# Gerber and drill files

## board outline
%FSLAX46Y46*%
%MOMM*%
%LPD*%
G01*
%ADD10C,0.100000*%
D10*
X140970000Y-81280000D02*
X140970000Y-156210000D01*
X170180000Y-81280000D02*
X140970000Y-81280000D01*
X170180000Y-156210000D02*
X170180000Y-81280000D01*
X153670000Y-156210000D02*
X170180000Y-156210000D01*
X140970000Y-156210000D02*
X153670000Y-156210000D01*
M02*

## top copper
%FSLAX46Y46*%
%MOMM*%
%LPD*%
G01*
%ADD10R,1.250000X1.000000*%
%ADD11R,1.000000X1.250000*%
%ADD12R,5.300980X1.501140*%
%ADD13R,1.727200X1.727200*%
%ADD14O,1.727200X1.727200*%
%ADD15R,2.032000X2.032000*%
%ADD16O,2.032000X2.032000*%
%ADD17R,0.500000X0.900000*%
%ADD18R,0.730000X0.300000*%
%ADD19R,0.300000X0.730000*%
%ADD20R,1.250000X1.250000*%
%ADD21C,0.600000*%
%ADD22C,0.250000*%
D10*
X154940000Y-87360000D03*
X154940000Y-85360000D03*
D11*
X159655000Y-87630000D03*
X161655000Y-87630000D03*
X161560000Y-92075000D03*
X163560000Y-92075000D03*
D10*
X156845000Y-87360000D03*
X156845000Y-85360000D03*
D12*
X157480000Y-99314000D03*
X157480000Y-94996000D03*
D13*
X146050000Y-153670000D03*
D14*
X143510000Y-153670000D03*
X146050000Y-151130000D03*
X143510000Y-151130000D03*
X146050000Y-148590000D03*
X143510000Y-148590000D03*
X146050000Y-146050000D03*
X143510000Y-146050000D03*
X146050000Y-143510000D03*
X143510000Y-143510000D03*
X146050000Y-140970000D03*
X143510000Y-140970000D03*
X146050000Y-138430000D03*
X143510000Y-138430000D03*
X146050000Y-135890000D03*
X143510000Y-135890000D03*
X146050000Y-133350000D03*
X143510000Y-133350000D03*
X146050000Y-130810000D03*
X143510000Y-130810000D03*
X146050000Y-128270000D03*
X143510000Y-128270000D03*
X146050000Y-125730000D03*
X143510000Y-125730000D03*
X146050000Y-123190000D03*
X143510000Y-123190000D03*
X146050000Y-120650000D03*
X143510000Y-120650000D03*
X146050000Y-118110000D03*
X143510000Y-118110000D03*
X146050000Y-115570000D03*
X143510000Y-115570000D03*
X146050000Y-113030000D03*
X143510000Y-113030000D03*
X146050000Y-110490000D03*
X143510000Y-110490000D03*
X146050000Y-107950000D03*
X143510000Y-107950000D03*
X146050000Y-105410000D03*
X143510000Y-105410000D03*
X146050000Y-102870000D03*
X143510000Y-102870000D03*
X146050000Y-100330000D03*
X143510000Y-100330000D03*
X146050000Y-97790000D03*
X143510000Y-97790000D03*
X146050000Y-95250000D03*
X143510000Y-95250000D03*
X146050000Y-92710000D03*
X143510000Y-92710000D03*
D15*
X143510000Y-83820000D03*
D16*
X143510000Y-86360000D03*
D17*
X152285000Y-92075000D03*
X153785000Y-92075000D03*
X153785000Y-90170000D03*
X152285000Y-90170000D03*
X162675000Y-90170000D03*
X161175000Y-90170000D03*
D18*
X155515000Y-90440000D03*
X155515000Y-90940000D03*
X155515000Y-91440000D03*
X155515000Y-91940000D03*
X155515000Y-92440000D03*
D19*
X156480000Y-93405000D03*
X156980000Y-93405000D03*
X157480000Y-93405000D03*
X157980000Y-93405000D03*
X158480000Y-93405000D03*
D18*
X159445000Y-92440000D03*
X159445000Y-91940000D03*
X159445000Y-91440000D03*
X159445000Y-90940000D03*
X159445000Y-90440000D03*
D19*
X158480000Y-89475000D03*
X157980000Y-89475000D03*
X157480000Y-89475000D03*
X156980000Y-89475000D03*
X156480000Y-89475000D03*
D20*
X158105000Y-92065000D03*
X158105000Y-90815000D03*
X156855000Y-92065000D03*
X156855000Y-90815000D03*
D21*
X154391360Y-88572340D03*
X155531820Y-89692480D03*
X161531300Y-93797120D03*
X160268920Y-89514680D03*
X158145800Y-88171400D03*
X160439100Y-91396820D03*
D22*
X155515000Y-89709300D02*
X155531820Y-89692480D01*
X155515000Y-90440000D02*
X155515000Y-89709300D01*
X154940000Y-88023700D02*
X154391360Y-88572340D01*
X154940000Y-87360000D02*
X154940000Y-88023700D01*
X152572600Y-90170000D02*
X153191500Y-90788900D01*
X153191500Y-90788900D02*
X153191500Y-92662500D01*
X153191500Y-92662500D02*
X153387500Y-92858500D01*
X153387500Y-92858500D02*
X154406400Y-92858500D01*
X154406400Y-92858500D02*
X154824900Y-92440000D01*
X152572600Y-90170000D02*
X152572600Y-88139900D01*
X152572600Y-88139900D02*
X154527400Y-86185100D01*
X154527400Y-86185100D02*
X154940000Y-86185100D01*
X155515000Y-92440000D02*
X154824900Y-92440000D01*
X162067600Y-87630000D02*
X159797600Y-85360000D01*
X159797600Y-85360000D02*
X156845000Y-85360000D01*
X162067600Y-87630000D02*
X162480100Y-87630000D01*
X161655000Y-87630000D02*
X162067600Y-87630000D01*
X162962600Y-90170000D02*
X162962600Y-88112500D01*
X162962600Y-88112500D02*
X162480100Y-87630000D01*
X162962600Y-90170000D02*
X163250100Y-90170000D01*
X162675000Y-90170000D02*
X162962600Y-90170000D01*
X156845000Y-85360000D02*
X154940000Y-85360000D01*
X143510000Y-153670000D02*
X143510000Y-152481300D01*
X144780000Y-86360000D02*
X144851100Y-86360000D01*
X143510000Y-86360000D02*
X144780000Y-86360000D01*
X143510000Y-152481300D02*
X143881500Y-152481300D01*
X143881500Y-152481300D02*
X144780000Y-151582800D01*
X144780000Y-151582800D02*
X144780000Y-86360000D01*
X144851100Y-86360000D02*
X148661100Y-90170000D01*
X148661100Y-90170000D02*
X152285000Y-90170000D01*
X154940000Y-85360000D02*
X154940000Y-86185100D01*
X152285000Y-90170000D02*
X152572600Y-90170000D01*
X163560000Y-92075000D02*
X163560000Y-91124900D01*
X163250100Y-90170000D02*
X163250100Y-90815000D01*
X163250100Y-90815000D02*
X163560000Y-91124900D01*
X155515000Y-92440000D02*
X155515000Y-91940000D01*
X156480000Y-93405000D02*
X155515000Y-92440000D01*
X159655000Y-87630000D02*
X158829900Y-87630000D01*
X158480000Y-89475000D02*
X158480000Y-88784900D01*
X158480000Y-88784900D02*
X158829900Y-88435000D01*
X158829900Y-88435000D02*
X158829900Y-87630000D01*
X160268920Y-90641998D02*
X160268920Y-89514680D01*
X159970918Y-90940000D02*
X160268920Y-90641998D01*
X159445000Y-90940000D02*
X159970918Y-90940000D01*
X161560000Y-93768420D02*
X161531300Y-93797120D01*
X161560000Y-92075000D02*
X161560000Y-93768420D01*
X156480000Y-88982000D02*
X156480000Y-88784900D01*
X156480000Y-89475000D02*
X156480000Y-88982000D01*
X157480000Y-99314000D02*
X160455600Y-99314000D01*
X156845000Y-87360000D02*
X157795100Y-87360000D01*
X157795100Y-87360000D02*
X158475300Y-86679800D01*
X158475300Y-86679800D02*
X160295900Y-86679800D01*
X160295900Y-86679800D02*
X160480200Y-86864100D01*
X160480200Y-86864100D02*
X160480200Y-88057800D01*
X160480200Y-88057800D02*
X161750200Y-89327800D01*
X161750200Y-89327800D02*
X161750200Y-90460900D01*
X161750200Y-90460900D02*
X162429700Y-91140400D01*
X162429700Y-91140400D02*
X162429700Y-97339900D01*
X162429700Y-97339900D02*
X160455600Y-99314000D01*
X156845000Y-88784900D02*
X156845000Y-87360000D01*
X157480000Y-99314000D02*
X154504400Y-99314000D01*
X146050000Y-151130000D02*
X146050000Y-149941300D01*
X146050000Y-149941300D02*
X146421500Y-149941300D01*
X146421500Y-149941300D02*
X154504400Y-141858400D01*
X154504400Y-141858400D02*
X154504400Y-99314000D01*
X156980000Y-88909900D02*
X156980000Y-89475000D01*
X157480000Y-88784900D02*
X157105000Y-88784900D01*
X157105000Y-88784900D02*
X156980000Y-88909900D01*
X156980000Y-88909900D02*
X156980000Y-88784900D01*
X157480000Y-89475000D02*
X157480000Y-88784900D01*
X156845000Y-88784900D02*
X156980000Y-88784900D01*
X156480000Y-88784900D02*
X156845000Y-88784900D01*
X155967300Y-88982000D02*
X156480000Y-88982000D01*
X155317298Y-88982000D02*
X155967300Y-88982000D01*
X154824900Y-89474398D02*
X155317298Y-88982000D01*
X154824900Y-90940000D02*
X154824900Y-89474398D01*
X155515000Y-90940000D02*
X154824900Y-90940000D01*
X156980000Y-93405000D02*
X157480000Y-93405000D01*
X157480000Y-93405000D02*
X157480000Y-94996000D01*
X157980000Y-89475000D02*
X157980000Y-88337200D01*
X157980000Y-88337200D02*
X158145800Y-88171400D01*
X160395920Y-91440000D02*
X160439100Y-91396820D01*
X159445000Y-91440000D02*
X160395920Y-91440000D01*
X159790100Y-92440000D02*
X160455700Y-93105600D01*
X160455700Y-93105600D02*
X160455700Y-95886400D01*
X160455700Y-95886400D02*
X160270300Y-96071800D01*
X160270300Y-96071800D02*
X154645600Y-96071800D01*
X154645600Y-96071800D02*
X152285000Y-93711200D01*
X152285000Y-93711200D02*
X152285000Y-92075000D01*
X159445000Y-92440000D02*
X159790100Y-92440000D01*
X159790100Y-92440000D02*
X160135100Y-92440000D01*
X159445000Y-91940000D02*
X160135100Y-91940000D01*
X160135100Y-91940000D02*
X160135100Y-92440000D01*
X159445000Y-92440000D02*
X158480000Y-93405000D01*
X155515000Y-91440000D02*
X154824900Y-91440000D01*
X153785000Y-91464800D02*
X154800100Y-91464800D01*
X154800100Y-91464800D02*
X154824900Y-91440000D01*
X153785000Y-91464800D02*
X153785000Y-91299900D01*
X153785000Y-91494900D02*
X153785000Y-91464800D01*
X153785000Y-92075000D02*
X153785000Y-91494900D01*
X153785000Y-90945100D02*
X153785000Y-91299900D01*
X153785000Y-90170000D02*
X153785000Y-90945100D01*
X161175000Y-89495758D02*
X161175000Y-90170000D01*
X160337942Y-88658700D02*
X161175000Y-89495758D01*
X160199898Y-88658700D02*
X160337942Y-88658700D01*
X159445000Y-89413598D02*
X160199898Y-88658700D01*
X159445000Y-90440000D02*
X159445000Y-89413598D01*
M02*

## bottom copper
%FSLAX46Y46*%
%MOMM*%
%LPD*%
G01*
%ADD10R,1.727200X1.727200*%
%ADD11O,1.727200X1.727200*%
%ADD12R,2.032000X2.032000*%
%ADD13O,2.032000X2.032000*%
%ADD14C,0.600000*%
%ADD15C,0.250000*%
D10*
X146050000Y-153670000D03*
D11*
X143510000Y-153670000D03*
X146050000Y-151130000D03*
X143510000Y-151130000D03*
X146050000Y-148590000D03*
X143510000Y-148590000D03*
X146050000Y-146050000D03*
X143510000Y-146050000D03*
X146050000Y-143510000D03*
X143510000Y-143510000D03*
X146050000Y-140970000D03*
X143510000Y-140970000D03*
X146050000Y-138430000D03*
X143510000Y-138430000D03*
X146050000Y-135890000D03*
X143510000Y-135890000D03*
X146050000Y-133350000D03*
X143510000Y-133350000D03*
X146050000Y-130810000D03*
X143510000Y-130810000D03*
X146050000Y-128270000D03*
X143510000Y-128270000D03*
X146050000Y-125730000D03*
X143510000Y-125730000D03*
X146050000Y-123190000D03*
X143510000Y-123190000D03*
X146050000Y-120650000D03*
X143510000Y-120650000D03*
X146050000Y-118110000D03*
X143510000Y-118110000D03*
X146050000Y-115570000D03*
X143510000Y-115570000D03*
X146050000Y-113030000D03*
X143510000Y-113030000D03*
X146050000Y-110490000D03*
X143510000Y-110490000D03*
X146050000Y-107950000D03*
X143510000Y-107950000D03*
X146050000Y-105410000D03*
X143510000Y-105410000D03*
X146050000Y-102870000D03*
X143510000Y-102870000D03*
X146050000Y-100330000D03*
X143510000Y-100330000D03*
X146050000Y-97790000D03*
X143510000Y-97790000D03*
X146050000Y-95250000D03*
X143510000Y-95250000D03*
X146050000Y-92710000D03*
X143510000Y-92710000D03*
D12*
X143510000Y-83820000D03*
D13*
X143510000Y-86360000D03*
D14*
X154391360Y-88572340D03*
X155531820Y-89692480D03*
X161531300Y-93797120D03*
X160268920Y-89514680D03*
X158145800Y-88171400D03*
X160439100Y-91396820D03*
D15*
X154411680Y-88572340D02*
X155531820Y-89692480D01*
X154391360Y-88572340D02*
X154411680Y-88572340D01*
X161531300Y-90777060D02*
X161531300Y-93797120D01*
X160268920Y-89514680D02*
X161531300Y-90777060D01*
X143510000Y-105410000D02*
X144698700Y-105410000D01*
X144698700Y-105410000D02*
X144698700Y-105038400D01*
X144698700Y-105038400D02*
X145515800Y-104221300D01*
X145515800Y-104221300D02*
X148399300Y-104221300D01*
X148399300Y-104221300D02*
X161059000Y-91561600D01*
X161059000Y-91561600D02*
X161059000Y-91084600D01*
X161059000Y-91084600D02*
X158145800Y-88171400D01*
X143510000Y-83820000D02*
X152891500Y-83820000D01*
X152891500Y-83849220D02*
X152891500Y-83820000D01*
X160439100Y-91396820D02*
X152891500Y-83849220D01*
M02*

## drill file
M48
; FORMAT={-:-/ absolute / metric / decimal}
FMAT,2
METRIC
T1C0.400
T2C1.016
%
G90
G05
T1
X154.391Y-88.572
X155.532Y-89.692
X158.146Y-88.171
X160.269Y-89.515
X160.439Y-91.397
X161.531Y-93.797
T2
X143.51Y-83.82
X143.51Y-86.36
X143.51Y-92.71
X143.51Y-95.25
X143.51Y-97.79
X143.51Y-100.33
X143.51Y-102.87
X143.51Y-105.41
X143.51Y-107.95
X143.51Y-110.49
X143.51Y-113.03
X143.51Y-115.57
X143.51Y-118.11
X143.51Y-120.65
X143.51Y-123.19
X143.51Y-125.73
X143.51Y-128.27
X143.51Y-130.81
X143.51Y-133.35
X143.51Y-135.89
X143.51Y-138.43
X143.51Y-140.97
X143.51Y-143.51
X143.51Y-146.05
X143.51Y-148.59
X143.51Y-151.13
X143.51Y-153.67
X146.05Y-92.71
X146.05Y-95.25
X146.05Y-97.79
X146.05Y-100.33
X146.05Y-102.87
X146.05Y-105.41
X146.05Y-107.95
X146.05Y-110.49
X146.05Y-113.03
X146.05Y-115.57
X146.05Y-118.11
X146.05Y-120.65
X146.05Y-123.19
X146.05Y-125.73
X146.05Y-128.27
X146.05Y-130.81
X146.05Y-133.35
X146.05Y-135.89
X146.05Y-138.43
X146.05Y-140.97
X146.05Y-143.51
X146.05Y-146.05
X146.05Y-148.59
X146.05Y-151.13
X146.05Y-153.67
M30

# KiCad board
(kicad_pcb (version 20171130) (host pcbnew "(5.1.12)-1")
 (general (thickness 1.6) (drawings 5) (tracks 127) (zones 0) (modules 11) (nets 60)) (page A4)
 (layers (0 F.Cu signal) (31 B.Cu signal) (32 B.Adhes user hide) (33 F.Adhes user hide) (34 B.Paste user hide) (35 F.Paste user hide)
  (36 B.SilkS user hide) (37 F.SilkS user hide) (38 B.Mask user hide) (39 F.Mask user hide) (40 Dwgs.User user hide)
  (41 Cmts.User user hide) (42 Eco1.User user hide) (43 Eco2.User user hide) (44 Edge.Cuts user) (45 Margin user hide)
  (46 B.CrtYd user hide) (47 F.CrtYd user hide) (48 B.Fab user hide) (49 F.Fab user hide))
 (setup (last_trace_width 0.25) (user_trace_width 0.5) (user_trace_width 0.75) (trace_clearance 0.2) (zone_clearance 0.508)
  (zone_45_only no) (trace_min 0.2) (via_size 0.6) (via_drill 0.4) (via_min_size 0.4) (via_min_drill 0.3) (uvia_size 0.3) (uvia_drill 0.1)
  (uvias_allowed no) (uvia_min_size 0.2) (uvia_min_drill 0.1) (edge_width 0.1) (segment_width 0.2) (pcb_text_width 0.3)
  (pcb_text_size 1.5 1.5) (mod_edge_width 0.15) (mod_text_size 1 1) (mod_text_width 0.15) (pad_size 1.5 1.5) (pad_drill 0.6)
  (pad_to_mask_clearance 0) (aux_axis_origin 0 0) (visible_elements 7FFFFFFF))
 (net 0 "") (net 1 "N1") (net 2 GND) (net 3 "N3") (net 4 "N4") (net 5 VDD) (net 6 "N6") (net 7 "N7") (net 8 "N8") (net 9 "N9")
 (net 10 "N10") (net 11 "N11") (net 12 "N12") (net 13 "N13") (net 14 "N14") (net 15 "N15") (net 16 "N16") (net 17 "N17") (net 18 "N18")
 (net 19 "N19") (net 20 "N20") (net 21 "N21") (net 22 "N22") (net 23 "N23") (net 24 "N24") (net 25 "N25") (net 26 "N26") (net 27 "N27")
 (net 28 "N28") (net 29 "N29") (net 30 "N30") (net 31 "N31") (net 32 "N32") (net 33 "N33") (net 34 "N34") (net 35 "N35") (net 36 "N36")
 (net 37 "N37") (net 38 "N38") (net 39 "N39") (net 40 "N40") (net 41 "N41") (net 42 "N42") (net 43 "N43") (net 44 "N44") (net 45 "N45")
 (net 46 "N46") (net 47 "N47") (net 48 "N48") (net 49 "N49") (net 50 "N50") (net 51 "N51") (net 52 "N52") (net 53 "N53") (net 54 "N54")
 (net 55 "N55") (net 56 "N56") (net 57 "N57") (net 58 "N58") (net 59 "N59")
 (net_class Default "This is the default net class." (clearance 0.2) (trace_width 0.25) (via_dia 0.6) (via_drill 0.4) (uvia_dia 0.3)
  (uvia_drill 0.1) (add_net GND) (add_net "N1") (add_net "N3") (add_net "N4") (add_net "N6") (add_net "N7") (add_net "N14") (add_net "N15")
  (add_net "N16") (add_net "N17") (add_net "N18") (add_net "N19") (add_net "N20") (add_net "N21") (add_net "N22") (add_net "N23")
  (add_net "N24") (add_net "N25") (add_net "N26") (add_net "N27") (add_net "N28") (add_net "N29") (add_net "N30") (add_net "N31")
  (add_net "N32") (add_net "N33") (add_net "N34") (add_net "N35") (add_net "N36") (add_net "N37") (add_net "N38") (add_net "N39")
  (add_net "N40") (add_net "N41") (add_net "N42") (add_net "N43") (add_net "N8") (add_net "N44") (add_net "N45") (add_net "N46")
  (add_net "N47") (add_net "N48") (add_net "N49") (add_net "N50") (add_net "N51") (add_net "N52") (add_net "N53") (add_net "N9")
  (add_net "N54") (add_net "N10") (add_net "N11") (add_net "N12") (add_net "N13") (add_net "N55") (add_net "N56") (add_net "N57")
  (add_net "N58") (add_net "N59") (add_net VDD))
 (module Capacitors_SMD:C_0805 (layer F.Cu) (at 154.94 86.36 90)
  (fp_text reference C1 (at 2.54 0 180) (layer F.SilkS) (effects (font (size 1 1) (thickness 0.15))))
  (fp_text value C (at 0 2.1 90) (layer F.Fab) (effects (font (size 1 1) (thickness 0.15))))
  (pad 1 smd rect (at -1 0 90) (size 1 1.25) (layers F.Cu F.Paste F.Mask) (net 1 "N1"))
  (pad 2 smd rect (at 1 0 90) (size 1 1.25) (layers F.Cu F.Paste F.Mask) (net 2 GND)))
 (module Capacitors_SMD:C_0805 (layer F.Cu) (at 160.655 87.63)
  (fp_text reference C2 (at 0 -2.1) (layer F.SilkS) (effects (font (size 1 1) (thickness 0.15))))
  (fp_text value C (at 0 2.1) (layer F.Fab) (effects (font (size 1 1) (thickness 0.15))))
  (pad 1 smd rect (at -1 0) (size 1 1.25) (layers F.Cu F.Paste F.Mask) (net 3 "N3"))
  (pad 2 smd rect (at 1 0) (size 1 1.25) (layers F.Cu F.Paste F.Mask) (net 2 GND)))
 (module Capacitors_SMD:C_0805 (layer F.Cu) (at 162.56 92.075)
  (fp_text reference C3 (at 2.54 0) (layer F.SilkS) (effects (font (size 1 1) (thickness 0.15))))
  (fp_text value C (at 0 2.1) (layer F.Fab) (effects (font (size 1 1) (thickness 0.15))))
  (pad 1 smd rect (at -1 0) (size 1 1.25) (layers F.Cu F.Paste F.Mask) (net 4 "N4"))
  (pad 2 smd rect (at 1 0) (size 1 1.25) (layers F.Cu F.Paste F.Mask) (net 2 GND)))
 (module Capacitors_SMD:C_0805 (layer F.Cu) (at 156.845 86.36 90)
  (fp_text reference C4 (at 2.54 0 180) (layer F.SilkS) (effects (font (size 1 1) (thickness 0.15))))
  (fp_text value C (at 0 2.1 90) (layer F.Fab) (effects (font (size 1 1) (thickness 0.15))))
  (pad 1 smd rect (at -1 0 90) (size 1 1.25) (layers F.Cu F.Paste F.Mask) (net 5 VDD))
  (pad 2 smd rect (at 1 0 90) (size 1 1.25) (layers F.Cu F.Paste F.Mask) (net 2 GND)))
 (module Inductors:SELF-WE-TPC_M (layer F.Cu) (at 157.48 97.155 90)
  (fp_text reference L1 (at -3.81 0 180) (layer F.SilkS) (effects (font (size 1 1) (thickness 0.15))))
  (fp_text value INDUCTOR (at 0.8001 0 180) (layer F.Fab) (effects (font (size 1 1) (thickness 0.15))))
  (pad 1 smd rect (at -2.159 0 90) (size 1.50114 5.30098) (layers F.Cu F.Paste F.Mask) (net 5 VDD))
  (pad 2 smd rect (at 2.159 0 90) (size 1.50114 5.30098) (layers F.Cu F.Paste F.Mask) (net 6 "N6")))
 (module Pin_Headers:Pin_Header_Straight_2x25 (layer F.Cu) (at 146.05 153.67 180)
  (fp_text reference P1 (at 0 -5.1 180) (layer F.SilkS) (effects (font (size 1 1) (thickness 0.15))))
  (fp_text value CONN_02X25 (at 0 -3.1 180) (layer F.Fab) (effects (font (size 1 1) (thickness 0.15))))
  (pad 1 thru_hole rect (at 0 0 180) (size 1.7272 1.7272) (drill 1.016) (layers *.Cu *.Mask F.SilkS) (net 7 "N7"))
  (pad 2 thru_hole oval (at 2.54 0 180) (size 1.7272 1.7272) (drill 1.016) (layers *.Cu *.Mask F.SilkS) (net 2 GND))
  (pad 3 thru_hole oval (at 0 2.54 180) (size 1.7272 1.7272) (drill 1.016) (layers *.Cu *.Mask F.SilkS) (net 5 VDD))
  (pad 4 thru_hole oval (at 2.54 2.54 180) (size 1.7272 1.7272) (drill 1.016) (layers *.Cu *.Mask F.SilkS) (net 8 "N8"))
  (pad 5 thru_hole oval (at 0 5.08 180) (size 1.7272 1.7272) (drill 1.016) (layers *.Cu *.Mask F.SilkS) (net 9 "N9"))
  (pad 6 thru_hole oval (at 2.54 5.08 180) (size 1.7272 1.7272) (drill 1.016) (layers *.Cu *.Mask F.SilkS) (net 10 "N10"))
  (pad 7 thru_hole oval (at 0 7.62 180) (size 1.7272 1.7272) (drill 1.016) (layers *.Cu *.Mask F.SilkS) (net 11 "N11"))
  (pad 8 thru_hole oval (at 2.54 7.62 180) (size 1.7272 1.7272) (drill 1.016) (layers *.Cu *.Mask F.SilkS) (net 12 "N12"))
  (pad 9 thru_hole oval (at 0 10.16 180) (size 1.7272 1.7272) (drill 1.016) (layers *.Cu *.Mask F.SilkS) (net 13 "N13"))
  (pad 10 thru_hole oval (at 2.54 10.16 180) (size 1.7272 1.7272) (drill 1.016) (layers *.Cu *.Mask F.SilkS) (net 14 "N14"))
  (pad 11 thru_hole oval (at 0 12.7 180) (size 1.7272 1.7272) (drill 1.016) (layers *.Cu *.Mask F.SilkS) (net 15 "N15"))
  (pad 12 thru_hole oval (at 2.54 12.7 180) (size 1.7272 1.7272) (drill 1.016) (layers *.Cu *.Mask F.SilkS) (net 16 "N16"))
  (pad 13 thru_hole oval (at 0 15.24 180) (size 1.7272 1.7272) (drill 1.016) (layers *.Cu *.Mask F.SilkS) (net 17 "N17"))
  (pad 14 thru_hole oval (at 2.54 15.24 180) (size 1.7272 1.7272) (drill 1.016) (layers *.Cu *.Mask F.SilkS) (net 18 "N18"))
  (pad 15 thru_hole oval (at 0 17.78 180) (size 1.7272 1.7272) (drill 1.016) (layers *.Cu *.Mask F.SilkS) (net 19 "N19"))
  (pad 16 thru_hole oval (at 2.54 17.78 180) (size 1.7272 1.7272) (drill 1.016) (layers *.Cu *.Mask F.SilkS) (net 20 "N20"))
  (pad 17 thru_hole oval (at 0 20.32 180) (size 1.7272 1.7272) (drill 1.016) (layers *.Cu *.Mask F.SilkS) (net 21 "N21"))
  (pad 18 thru_hole oval (at 2.54 20.32 180) (size 1.7272 1.7272) (drill 1.016) (layers *.Cu *.Mask F.SilkS) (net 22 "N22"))
  (pad 19 thru_hole oval (at 0 22.86 180) (size 1.7272 1.7272) (drill 1.016) (layers *.Cu *.Mask F.SilkS) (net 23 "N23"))
  (pad 20 thru_hole oval (at 2.54 22.86 180) (size 1.7272 1.7272) (drill 1.016) (layers *.Cu *.Mask F.SilkS) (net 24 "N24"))
  (pad 21 thru_hole oval (at 0 25.4 180) (size 1.7272 1.7272) (drill 1.016) (layers *.Cu *.Mask F.SilkS) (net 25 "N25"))
  (pad 22 thru_hole oval (at 2.54 25.4 180) (size 1.7272 1.7272) (drill 1.016) (layers *.Cu *.Mask F.SilkS) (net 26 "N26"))
  (pad 23 thru_hole oval (at 0 27.94 180) (size 1.7272 1.7272) (drill 1.016) (layers *.Cu *.Mask F.SilkS) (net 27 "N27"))
  (pad 24 thru_hole oval (at 2.54 27.94 180) (size 1.7272 1.7272) (drill 1.016) (layers *.Cu *.Mask F.SilkS) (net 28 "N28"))
  (pad 25 thru_hole oval (at 0 30.48 180) (size 1.7272 1.7272) (drill 1.016) (layers *.Cu *.Mask F.SilkS) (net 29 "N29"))
  (pad 26 thru_hole oval (at 2.54 30.48 180) (size 1.7272 1.7272) (drill 1.016) (layers *.Cu *.Mask F.SilkS) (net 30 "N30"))
  (pad 27 thru_hole oval (at 0 33.02 180) (size 1.7272 1.7272) (drill 1.016) (layers *.Cu *.Mask F.SilkS) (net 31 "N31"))
  (pad 28 thru_hole oval (at 2.54 33.02 180) (size 1.7272 1.7272) (drill 1.016) (layers *.Cu *.Mask F.SilkS) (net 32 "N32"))
  (pad 29 thru_hole oval (at 0 35.56 180) (size 1.7272 1.7272) (drill 1.016) (layers *.Cu *.Mask F.SilkS) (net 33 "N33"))
  (pad 30 thru_hole oval (at 2.54 35.56 180) (size 1.7272 1.7272) (drill 1.016) (layers *.Cu *.Mask F.SilkS) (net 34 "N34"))
  (pad 31 thru_hole oval (at 0 38.1 180) (size 1.7272 1.7272) (drill 1.016) (layers *.Cu *.Mask F.SilkS) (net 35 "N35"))
  (pad 32 thru_hole oval (at 2.54 38.1 180) (size 1.7272 1.7272) (drill 1.016) (layers *.Cu *.Mask F.SilkS) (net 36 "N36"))
  (pad 33 thru_hole oval (at 0 40.64 180) (size 1.7272 1.7272) (drill 1.016) (layers *.Cu *.Mask F.SilkS) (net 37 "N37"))
  (pad 34 thru_hole oval (at 2.54 40.64 180) (size 1.7272 1.7272) (drill 1.016) (layers *.Cu *.Mask F.SilkS) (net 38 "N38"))
  (pad 35 thru_hole oval (at 0 43.18 180) (size 1.7272 1.7272) (drill 1.016) (layers *.Cu *.Mask F.SilkS) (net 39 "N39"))
  (pad 36 thru_hole oval (at 2.54 43.18 180) (size 1.7272 1.7272) (drill 1.016) (layers *.Cu *.Mask F.SilkS) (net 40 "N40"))
  (pad 37 thru_hole oval (at 0 45.72 180) (size 1.7272 1.7272) (drill 1.016) (layers *.Cu *.Mask F.SilkS) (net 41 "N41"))
  (pad 38 thru_hole oval (at 2.54 45.72 180) (size 1.7272 1.7272) (drill 1.016) (layers *.Cu *.Mask F.SilkS) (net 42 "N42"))
  (pad 39 thru_hole oval (at 0 48.26 180) (size 1.7272 1.7272) (drill 1.016) (layers *.Cu *.Mask F.SilkS) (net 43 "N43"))
  (pad 40 thru_hole oval (at 2.54 48.26 180) (size 1.7272 1.7272) (drill 1.016) (layers *.Cu *.Mask F.SilkS) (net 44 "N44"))
  (pad 41 thru_hole oval (at 0 50.8 180) (size 1.7272 1.7272) (drill 1.016) (layers *.Cu *.Mask F.SilkS) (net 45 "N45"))
  (pad 42 thru_hole oval (at 2.54 50.8 180) (size 1.7272 1.7272) (drill 1.016) (layers *.Cu *.Mask F.SilkS) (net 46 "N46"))
  (pad 43 thru_hole oval (at 0 53.34 180) (size 1.7272 1.7272) (drill 1.016) (layers *.Cu *.Mask F.SilkS) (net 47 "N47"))
  (pad 44 thru_hole oval (at 2.54 53.34 180) (size 1.7272 1.7272) (drill 1.016) (layers *.Cu *.Mask F.SilkS) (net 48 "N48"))
  (pad 45 thru_hole oval (at 0 55.88 180) (size 1.7272 1.7272) (drill 1.016) (layers *.Cu *.Mask F.SilkS) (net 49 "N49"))
  (pad 46 thru_hole oval (at 2.54 55.88 180) (size 1.7272 1.7272) (drill 1.016) (layers *.Cu *.Mask F.SilkS) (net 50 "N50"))
  (pad 47 thru_hole oval (at 0 58.42 180) (size 1.7272 1.7272) (drill 1.016) (layers *.Cu *.Mask F.SilkS) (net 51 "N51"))
  (pad 48 thru_hole oval (at 2.54 58.42 180) (size 1.7272 1.7272) (drill 1.016) (layers *.Cu *.Mask F.SilkS) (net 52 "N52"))
  (pad 49 thru_hole oval (at 0 60.96 180) (size 1.7272 1.7272) (drill 1.016) (layers *.Cu *.Mask F.SilkS) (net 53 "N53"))
  (pad 50 thru_hole oval (at 2.54 60.96 180) (size 1.7272 1.7272) (drill 1.016) (layers *.Cu *.Mask F.SilkS) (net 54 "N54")))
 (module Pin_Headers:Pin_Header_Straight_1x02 (layer F.Cu) (at 143.51 83.82)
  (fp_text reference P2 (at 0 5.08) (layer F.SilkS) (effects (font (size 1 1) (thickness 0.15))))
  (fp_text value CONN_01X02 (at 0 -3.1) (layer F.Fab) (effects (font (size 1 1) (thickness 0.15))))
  (pad 1 thru_hole rect (at 0 0) (size 2.032 2.032) (drill 1.016) (layers *.Cu *.Mask F.SilkS) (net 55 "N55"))
  (pad 2 thru_hole oval (at 0 2.54) (size 2.032 2.032) (drill 1.016) (layers *.Cu *.Mask F.SilkS) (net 2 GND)))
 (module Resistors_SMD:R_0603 (layer F.Cu) (at 153.035 92.075)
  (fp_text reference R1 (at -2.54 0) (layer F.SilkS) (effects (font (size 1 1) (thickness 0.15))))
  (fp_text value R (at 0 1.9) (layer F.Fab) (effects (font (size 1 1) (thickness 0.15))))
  (pad 1 smd rect (at -0.75 0) (size 0.5 0.9) (layers F.Cu F.Paste F.Mask) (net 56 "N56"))
  (pad 2 smd rect (at 0.75 0) (size 0.5 0.9) (layers F.Cu F.Paste F.Mask) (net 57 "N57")))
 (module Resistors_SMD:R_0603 (layer F.Cu) (at 153.035 90.17 180)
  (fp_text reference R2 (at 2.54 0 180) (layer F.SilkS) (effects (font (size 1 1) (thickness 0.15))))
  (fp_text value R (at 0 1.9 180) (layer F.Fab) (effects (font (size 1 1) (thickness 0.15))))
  (pad 1 smd rect (at -0.75 0 180) (size 0.5 0.9) (layers F.Cu F.Paste F.Mask) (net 57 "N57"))
  (pad 2 smd rect (at 0.75 0 180) (size 0.5 0.9) (layers F.Cu F.Paste F.Mask) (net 2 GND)))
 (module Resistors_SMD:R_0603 (layer F.Cu) (at 161.925 90.17 180)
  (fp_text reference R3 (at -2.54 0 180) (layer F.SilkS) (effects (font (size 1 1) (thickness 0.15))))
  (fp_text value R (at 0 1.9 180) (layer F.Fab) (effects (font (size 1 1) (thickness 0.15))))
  (pad 1 smd rect (at -0.75 0 180) (size 0.5 0.9) (layers F.Cu F.Paste F.Mask) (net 2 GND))
  (pad 2 smd rect (at 0.75 0 180) (size 0.5 0.9) (layers F.Cu F.Paste F.Mask) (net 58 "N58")))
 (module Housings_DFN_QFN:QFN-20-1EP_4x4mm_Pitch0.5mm (layer F.Cu) (at 157.48 91.44)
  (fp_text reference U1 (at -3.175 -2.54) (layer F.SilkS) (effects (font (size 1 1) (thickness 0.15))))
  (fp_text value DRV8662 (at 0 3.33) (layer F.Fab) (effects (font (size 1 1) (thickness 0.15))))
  (pad 1 smd rect (at -1.965 -1) (size 0.73 0.3) (layers F.Cu F.Paste F.Mask) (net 1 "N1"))
  (pad 2 smd rect (at -1.965 -0.5) (size 0.73 0.3) (layers F.Cu F.Paste F.Mask) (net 5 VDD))
  (pad 3 smd rect (at -1.965 0) (size 0.73 0.3) (layers F.Cu F.Paste F.Mask) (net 57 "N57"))
  (pad 4 smd rect (at -1.965 0.5) (size 0.73 0.3) (layers F.Cu F.Paste F.Mask) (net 2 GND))
  (pad 5 smd rect (at -1.965 1) (size 0.73 0.3) (layers F.Cu F.Paste F.Mask) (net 2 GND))
  (pad 6 smd rect (at -1 1.965 90) (size 0.73 0.3) (layers F.Cu F.Paste F.Mask) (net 2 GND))
  (pad 7 smd rect (at -0.5 1.965 90) (size 0.73 0.3) (layers F.Cu F.Paste F.Mask) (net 6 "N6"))
  (pad 8 smd rect (at 0 1.965 90) (size 0.73 0.3) (layers F.Cu F.Paste F.Mask) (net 6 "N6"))
  (pad 9 smd rect (at 0.5 1.965 90) (size 0.73 0.3) (layers F.Cu F.Paste F.Mask) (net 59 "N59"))
  (pad 10 smd rect (at 1 1.965 90) (size 0.73 0.3) (layers F.Cu F.Paste F.Mask) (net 56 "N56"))
  (pad 11 smd rect (at 1.965 1) (size 0.73 0.3) (layers F.Cu F.Paste F.Mask) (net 56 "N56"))
  (pad 12 smd rect (at 1.965 0.5) (size 0.73 0.3) (layers F.Cu F.Paste F.Mask) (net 56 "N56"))
  (pad 13 smd rect (at 1.965 0) (size 0.73 0.3) (layers F.Cu F.Paste F.Mask) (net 55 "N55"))
  (pad 14 smd rect (at 1.965 -0.5) (size 0.73 0.3) (layers F.Cu F.Paste F.Mask) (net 4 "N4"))
  (pad 15 smd rect (at 1.965 -1) (size 0.73 0.3) (layers F.Cu F.Paste F.Mask) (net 58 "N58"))
  (pad 16 smd rect (at 1 -1.965 90) (size 0.73 0.3) (layers F.Cu F.Paste F.Mask) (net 3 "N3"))
  (pad 17 smd rect (at 0.5 -1.965 90) (size 0.73 0.3) (layers F.Cu F.Paste F.Mask) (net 44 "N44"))
  (pad 18 smd rect (at 0 -1.965 90) (size 0.73 0.3) (layers F.Cu F.Paste F.Mask) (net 5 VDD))
  (pad 19 smd rect (at -0.5 -1.965 90) (size 0.73 0.3) (layers F.Cu F.Paste F.Mask) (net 5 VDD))
  (pad 20 smd rect (at -1 -1.965 90) (size 0.73 0.3) (layers F.Cu F.Paste F.Mask) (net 5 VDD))
  (pad 21 smd rect (at 0.625 0.625) (size 1.25 1.25) (layers F.Cu F.Paste F.Mask) (solder_paste_margin_ratio -0.2))
  (pad 21 smd rect (at 0.625 -0.625) (size 1.25 1.25) (layers F.Cu F.Paste F.Mask) (solder_paste_margin_ratio -0.2))
  (pad 21 smd rect (at -0.625 0.625) (size 1.25 1.25) (layers F.Cu F.Paste F.Mask) (solder_paste_margin_ratio -0.2))
  (pad 21 smd rect (at -0.625 -0.625) (size 1.25 1.25) (layers F.Cu F.Paste F.Mask) (solder_paste_margin_ratio -0.2)))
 (gr_line (start 140.97 81.28) (end 140.97 156.21) (angle 90) (layer Edge.Cuts) (width 0.1))
 (gr_line (start 170.18 81.28) (end 140.97 81.28) (angle 90) (layer Edge.Cuts) (width 0.1))
 (gr_line (start 170.18 156.21) (end 170.18 81.28) (angle 90) (layer Edge.Cuts) (width 0.1))
 (gr_line (start 153.67 156.21) (end 170.18 156.21) (angle 90) (layer Edge.Cuts) (width 0.1))
 (gr_line (start 140.97 156.21) (end 153.67 156.21) (angle 90) (layer Edge.Cuts) (width 0.1))
 (via (at 154.39136 88.57234) (size 0.6) (drill 0.4) (layers F.Cu B.Cu) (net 1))
 (via (at 155.53182 89.69248) (size 0.6) (drill 0.4) (layers F.Cu B.Cu) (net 1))
 (segment (start 155.515 89.7093) (end 155.53182 89.69248) (width 0.25) (layer F.Cu) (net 1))
 (segment (start 155.515 90.44) (end 155.515 89.7093) (width 0.25) (layer F.Cu) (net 1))
 (segment (start 154.94 88.0237) (end 154.39136 88.57234) (width 0.25) (layer F.Cu) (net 1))
 (segment (start 154.94 87.36) (end 154.94 88.0237) (width 0.25) (layer F.Cu) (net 1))
 (segment (start 154.41168 88.57234) (end 155.53182 89.69248) (width 0.25) (layer B.Cu) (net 1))
 (segment (start 154.39136 88.57234) (end 154.41168 88.57234) (width 0.25) (layer B.Cu) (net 1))
 (via (at 161.5313 93.79712) (size 0.6) (drill 0.4) (layers F.Cu B.Cu) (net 4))
 (via (at 160.26892 89.51468) (size 0.6) (drill 0.4) (layers F.Cu B.Cu) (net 4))
 (segment (start 152.5726 90.17) (end 153.1915 90.7889) (width 0.25) (layer F.Cu) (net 2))
 (segment (start 153.1915 90.7889) (end 153.1915 92.6625) (width 0.25) (layer F.Cu) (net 2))
 (segment (start 153.1915 92.6625) (end 153.3875 92.8585) (width 0.25) (layer F.Cu) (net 2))
 (segment (start 153.3875 92.8585) (end 154.4064 92.8585) (width 0.25) (layer F.Cu) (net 2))
 (segment (start 154.4064 92.8585) (end 154.8249 92.44) (width 0.25) (layer F.Cu) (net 2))
 (segment (start 152.5726 90.17) (end 152.5726 88.1399) (width 0.25) (layer F.Cu) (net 2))
 (segment (start 152.5726 88.1399) (end 154.5274 86.1851) (width 0.25) (layer F.Cu) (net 2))
 (segment (start 154.5274 86.1851) (end 154.94 86.1851) (width 0.25) (layer F.Cu) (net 2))
 (segment (start 155.515 92.44) (end 154.8249 92.44) (width 0.25) (layer F.Cu) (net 2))
 (segment (start 162.0676 87.63) (end 159.7976 85.36) (width 0.25) (layer F.Cu) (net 2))
 (segment (start 159.7976 85.36) (end 156.845 85.36) (width 0.25) (layer F.Cu) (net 2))
 (segment (start 162.0676 87.63) (end 162.4801 87.63) (width 0.25) (layer F.Cu) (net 2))
 (segment (start 161.655 87.63) (end 162.0676 87.63) (width 0.25) (layer F.Cu) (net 2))
 (segment (start 162.9626 90.17) (end 162.9626 88.1125) (width 0.25) (layer F.Cu) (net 2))
 (segment (start 162.9626 88.1125) (end 162.4801 87.63) (width 0.25) (layer F.Cu) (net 2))
 (segment (start 162.9626 90.17) (end 163.2501 90.17) (width 0.25) (layer F.Cu) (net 2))
 (segment (start 162.675 90.17) (end 162.9626 90.17) (width 0.25) (layer F.Cu) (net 2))
 (segment (start 156.845 85.36) (end 154.94 85.36) (width 0.25) (layer F.Cu) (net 2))
 (segment (start 143.51 153.67) (end 143.51 152.4813) (width 0.25) (layer F.Cu) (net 2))
 (segment (start 144.78 86.36) (end 144.8511 86.36) (width 0.25) (layer F.Cu) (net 2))
 (segment (start 143.51 86.36) (end 144.78 86.36) (width 0.25) (layer F.Cu) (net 2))
 (segment (start 143.51 152.4813) (end 143.8815 152.4813) (width 0.25) (layer F.Cu) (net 2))
 (segment (start 143.8815 152.4813) (end 144.78 151.5828) (width 0.25) (layer F.Cu) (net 2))
 (segment (start 144.78 151.5828) (end 144.78 86.36) (width 0.25) (layer F.Cu) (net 2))
 (segment (start 144.8511 86.36) (end 148.6611 90.17) (width 0.25) (layer F.Cu) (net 2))
 (segment (start 148.6611 90.17) (end 152.285 90.17) (width 0.25) (layer F.Cu) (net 2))
 (segment (start 154.94 85.36) (end 154.94 86.1851) (width 0.25) (layer F.Cu) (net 2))
 (segment (start 152.285 90.17) (end 152.5726 90.17) (width 0.25) (layer F.Cu) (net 2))
 (segment (start 163.56 92.075) (end 163.56 91.1249) (width 0.25) (layer F.Cu) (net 2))
 (segment (start 163.2501 90.17) (end 163.2501 90.815) (width 0.25) (layer F.Cu) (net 2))
 (segment (start 163.2501 90.815) (end 163.56 91.1249) (width 0.25) (layer F.Cu) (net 2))
 (segment (start 155.515 92.44) (end 155.515 91.94) (width 0.25) (layer F.Cu) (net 2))
 (segment (start 156.48 93.405) (end 155.515 92.44) (width 0.25) (layer F.Cu) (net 2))
 (segment (start 159.655 87.63) (end 158.8299 87.63) (width 0.25) (layer F.Cu) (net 3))
 (segment (start 158.48 89.475) (end 158.48 88.7849) (width 0.25) (layer F.Cu) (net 3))
 (segment (start 158.48 88.7849) (end 158.8299 88.435) (width 0.25) (layer F.Cu) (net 3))
 (segment (start 158.8299 88.435) (end 158.8299 87.63) (width 0.25) (layer F.Cu) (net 3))
 (segment (start 160.26892 90.641998) (end 160.26892 89.51468) (width 0.25) (layer F.Cu) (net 4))
 (segment (start 159.970918 90.94) (end 160.26892 90.641998) (width 0.25) (layer F.Cu) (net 4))
 (segment (start 159.445 90.94) (end 159.970918 90.94) (width 0.25) (layer F.Cu) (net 4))
 (segment (start 161.56 93.76842) (end 161.5313 93.79712) (width 0.25) (layer F.Cu) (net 4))
 (segment (start 161.56 92.075) (end 161.56 93.76842) (width 0.25) (layer F.Cu) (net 4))
 (segment (start 161.5313 90.77706) (end 161.5313 93.79712) (width 0.25) (layer B.Cu) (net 4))
 (segment (start 160.26892 89.51468) (end 161.5313 90.77706) (width 0.25) (layer B.Cu) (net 4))
 (segment (start 156.48 88.982) (end 156.48 88.7849) (width 0.25) (layer F.Cu) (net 5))
 (segment (start 156.48 89.475) (end 156.48 88.982) (width 0.25) (layer F.Cu) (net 5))
 (segment (start 157.48 99.314) (end 160.4556 99.314) (width 0.25) (layer F.Cu) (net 5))
 (segment (start 156.845 87.36) (end 157.7951 87.36) (width 0.25) (layer F.Cu) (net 5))
 (segment (start 157.7951 87.36) (end 158.4753 86.6798) (width 0.25) (layer F.Cu) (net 5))
 (segment (start 158.4753 86.6798) (end 160.2959 86.6798) (width 0.25) (layer F.Cu) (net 5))
 (segment (start 160.2959 86.6798) (end 160.4802 86.8641) (width 0.25) (layer F.Cu) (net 5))
 (segment (start 160.4802 86.8641) (end 160.4802 88.0578) (width 0.25) (layer F.Cu) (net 5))
 (segment (start 160.4802 88.0578) (end 161.7502 89.3278) (width 0.25) (layer F.Cu) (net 5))
 (segment (start 161.7502 89.3278) (end 161.7502 90.4609) (width 0.25) (layer F.Cu) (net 5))
 (segment (start 161.7502 90.4609) (end 162.4297 91.1404) (width 0.25) (layer F.Cu) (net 5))
 (segment (start 162.4297 91.1404) (end 162.4297 97.3399) (width 0.25) (layer F.Cu) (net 5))
 (segment (start 162.4297 97.3399) (end 160.4556 99.314) (width 0.25) (layer F.Cu) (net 5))
 (segment (start 156.845 88.7849) (end 156.845 87.36) (width 0.25) (layer F.Cu) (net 5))
 (segment (start 157.48 99.314) (end 154.5044 99.314) (width 0.25) (layer F.Cu) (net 5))
 (segment (start 146.05 151.13) (end 146.05 149.9413) (width 0.25) (layer F.Cu) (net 5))
 (segment (start 146.05 149.9413) (end 146.4215 149.9413) (width 0.25) (layer F.Cu) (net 5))
 (segment (start 146.4215 149.9413) (end 154.5044 141.8584) (width 0.25) (layer F.Cu) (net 5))
 (segment (start 154.5044 141.8584) (end 154.5044 99.314) (width 0.25) (layer F.Cu) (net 5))
 (segment (start 156.98 88.9099) (end 156.98 89.475) (width 0.25) (layer F.Cu) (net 5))
 (segment (start 157.48 88.7849) (end 157.105 88.7849) (width 0.25) (layer F.Cu) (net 5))
 (segment (start 157.105 88.7849) (end 156.98 88.9099) (width 0.25) (layer F.Cu) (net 5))
 (segment (start 156.98 88.9099) (end 156.98 88.7849) (width 0.25) (layer F.Cu) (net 5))
 (segment (start 157.48 89.475) (end 157.48 88.7849) (width 0.25) (layer F.Cu) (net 5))
 (segment (start 156.845 88.7849) (end 156.98 88.7849) (width 0.25) (layer F.Cu) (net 5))
 (segment (start 156.48 88.7849) (end 156.845 88.7849) (width 0.25) (layer F.Cu) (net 5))
 (segment (start 155.9673 88.982) (end 156.48 88.982) (width 0.25) (layer F.Cu) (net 5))
 (segment (start 155.317298 88.982) (end 155.9673 88.982) (width 0.25) (layer F.Cu) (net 5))
 (segment (start 154.8249 89.474398) (end 155.317298 88.982) (width 0.25) (layer F.Cu) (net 5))
 (segment (start 154.8249 90.94) (end 154.8249 89.474398) (width 0.25) (layer F.Cu) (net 5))
 (segment (start 155.515 90.94) (end 154.8249 90.94) (width 0.25) (layer F.Cu) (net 5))
 (segment (start 156.98 93.405) (end 157.48 93.405) (width 0.25) (layer F.Cu) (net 6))
 (segment (start 157.48 93.405) (end 157.48 94.996) (width 0.25) (layer F.Cu) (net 6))
 (segment (start 143.51 105.41) (end 144.6987 105.41) (width 0.25) (layer B.Cu) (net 44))
 (segment (start 157.98 89.475) (end 157.98 88.3372) (width 0.25) (layer F.Cu) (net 44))
 (segment (start 157.98 88.3372) (end 158.1458 88.1714) (width 0.25) (layer F.Cu) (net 44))
 (segment (start 144.6987 105.41) (end 144.6987 105.0384) (width 0.25) (layer B.Cu) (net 44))
 (segment (start 144.6987 105.0384) (end 145.5158 104.2213) (width 0.25) (layer B.Cu) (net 44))
 (segment (start 145.5158 104.2213) (end 148.3993 104.2213) (width 0.25) (layer B.Cu) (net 44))
 (segment (start 148.3993 104.2213) (end 161.059 91.5616) (width 0.25) (layer B.Cu) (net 44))
 (segment (start 161.059 91.5616) (end 161.059 91.0846) (width 0.25) (layer B.Cu) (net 44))
 (segment (start 161.059 91.0846) (end 158.1458 88.1714) (width 0.25) (layer B.Cu) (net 44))
 (via (at 158.1458 88.1714) (size 0.6) (layers F.Cu B.Cu) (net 44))
 (segment (start 143.51 83.82) (end 152.8915 83.82) (width 0.25) (layer B.Cu) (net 55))
 (via (at 160.4391 91.39682) (size 0.6) (layers F.Cu B.Cu) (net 55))
 (segment (start 160.39592 91.44) (end 160.4391 91.39682) (width 0.25) (layer F.Cu) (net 55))
 (segment (start 159.445 91.44) (end 160.39592 91.44) (width 0.25) (layer F.Cu) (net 55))
 (segment (start 152.8915 83.84922) (end 152.8915 83.82) (width 0.25) (layer B.Cu) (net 55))
 (segment (start 160.4391 91.39682) (end 152.8915 83.84922) (width 0.25) (layer B.Cu) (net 55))
 (segment (start 159.7901 92.44) (end 160.4557 93.1056) (width 0.25) (layer F.Cu) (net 56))
 (segment (start 160.4557 93.1056) (end 160.4557 95.8864) (width 0.25) (layer F.Cu) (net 56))
 (segment (start 160.4557 95.8864) (end 160.2703 96.0718) (width 0.25) (layer F.Cu) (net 56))
 (segment (start 160.2703 96.0718) (end 154.6456 96.0718) (width 0.25) (layer F.Cu) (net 56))
 (segment (start 154.6456 96.0718) (end 152.285 93.7112) (width 0.25) (layer F.Cu) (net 56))
 (segment (start 152.285 93.7112) (end 152.285 92.075) (width 0.25) (layer F.Cu) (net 56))
 (segment (start 159.445 92.44) (end 159.7901 92.44) (width 0.25) (layer F.Cu) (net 56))
 (segment (start 159.7901 92.44) (end 160.1351 92.44) (width 0.25) (layer F.Cu) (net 56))
 (segment (start 159.445 91.94) (end 160.1351 91.94) (width 0.25) (layer F.Cu) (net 56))
 (segment (start 160.1351 91.94) (end 160.1351 92.44) (width 0.25) (layer F.Cu) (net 56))
 (segment (start 159.445 92.44) (end 158.48 93.405) (width 0.25) (layer F.Cu) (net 56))
 (segment (start 155.515 91.44) (end 154.8249 91.44) (width 0.25) (layer F.Cu) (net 57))
 (segment (start 153.785 91.4648) (end 154.8001 91.4648) (width 0.25) (layer F.Cu) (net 57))
 (segment (start 154.8001 91.4648) (end 154.8249 91.44) (width 0.25) (layer F.Cu) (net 57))
 (segment (start 153.785 91.4648) (end 153.785 91.2999) (width 0.25) (layer F.Cu) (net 57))
 (segment (start 153.785 91.4949) (end 153.785 91.4648) (width 0.25) (layer F.Cu) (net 57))
 (segment (start 153.785 92.075) (end 153.785 91.4949) (width 0.25) (layer F.Cu) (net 57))
 (segment (start 153.785 90.9451) (end 153.785 91.2999) (width 0.25) (layer F.Cu) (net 57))
 (segment (start 153.785 90.17) (end 153.785 90.9451) (width 0.25) (layer F.Cu) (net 57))
 (segment (start 161.175 89.495758) (end 161.175 90.17) (width 0.25) (layer F.Cu) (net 58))
 (segment (start 160.337942 88.6587) (end 161.175 89.495758) (width 0.25) (layer F.Cu) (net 58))
 (segment (start 160.199898 88.6587) (end 160.337942 88.6587) (width 0.25) (layer F.Cu) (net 58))
 (segment (start 159.445 89.413598) (end 160.199898 88.6587) (width 0.25) (layer F.Cu) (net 58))
 (segment (start 159.445 90.44) (end 159.445 89.413598) (width 0.25) (layer F.Cu) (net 58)))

